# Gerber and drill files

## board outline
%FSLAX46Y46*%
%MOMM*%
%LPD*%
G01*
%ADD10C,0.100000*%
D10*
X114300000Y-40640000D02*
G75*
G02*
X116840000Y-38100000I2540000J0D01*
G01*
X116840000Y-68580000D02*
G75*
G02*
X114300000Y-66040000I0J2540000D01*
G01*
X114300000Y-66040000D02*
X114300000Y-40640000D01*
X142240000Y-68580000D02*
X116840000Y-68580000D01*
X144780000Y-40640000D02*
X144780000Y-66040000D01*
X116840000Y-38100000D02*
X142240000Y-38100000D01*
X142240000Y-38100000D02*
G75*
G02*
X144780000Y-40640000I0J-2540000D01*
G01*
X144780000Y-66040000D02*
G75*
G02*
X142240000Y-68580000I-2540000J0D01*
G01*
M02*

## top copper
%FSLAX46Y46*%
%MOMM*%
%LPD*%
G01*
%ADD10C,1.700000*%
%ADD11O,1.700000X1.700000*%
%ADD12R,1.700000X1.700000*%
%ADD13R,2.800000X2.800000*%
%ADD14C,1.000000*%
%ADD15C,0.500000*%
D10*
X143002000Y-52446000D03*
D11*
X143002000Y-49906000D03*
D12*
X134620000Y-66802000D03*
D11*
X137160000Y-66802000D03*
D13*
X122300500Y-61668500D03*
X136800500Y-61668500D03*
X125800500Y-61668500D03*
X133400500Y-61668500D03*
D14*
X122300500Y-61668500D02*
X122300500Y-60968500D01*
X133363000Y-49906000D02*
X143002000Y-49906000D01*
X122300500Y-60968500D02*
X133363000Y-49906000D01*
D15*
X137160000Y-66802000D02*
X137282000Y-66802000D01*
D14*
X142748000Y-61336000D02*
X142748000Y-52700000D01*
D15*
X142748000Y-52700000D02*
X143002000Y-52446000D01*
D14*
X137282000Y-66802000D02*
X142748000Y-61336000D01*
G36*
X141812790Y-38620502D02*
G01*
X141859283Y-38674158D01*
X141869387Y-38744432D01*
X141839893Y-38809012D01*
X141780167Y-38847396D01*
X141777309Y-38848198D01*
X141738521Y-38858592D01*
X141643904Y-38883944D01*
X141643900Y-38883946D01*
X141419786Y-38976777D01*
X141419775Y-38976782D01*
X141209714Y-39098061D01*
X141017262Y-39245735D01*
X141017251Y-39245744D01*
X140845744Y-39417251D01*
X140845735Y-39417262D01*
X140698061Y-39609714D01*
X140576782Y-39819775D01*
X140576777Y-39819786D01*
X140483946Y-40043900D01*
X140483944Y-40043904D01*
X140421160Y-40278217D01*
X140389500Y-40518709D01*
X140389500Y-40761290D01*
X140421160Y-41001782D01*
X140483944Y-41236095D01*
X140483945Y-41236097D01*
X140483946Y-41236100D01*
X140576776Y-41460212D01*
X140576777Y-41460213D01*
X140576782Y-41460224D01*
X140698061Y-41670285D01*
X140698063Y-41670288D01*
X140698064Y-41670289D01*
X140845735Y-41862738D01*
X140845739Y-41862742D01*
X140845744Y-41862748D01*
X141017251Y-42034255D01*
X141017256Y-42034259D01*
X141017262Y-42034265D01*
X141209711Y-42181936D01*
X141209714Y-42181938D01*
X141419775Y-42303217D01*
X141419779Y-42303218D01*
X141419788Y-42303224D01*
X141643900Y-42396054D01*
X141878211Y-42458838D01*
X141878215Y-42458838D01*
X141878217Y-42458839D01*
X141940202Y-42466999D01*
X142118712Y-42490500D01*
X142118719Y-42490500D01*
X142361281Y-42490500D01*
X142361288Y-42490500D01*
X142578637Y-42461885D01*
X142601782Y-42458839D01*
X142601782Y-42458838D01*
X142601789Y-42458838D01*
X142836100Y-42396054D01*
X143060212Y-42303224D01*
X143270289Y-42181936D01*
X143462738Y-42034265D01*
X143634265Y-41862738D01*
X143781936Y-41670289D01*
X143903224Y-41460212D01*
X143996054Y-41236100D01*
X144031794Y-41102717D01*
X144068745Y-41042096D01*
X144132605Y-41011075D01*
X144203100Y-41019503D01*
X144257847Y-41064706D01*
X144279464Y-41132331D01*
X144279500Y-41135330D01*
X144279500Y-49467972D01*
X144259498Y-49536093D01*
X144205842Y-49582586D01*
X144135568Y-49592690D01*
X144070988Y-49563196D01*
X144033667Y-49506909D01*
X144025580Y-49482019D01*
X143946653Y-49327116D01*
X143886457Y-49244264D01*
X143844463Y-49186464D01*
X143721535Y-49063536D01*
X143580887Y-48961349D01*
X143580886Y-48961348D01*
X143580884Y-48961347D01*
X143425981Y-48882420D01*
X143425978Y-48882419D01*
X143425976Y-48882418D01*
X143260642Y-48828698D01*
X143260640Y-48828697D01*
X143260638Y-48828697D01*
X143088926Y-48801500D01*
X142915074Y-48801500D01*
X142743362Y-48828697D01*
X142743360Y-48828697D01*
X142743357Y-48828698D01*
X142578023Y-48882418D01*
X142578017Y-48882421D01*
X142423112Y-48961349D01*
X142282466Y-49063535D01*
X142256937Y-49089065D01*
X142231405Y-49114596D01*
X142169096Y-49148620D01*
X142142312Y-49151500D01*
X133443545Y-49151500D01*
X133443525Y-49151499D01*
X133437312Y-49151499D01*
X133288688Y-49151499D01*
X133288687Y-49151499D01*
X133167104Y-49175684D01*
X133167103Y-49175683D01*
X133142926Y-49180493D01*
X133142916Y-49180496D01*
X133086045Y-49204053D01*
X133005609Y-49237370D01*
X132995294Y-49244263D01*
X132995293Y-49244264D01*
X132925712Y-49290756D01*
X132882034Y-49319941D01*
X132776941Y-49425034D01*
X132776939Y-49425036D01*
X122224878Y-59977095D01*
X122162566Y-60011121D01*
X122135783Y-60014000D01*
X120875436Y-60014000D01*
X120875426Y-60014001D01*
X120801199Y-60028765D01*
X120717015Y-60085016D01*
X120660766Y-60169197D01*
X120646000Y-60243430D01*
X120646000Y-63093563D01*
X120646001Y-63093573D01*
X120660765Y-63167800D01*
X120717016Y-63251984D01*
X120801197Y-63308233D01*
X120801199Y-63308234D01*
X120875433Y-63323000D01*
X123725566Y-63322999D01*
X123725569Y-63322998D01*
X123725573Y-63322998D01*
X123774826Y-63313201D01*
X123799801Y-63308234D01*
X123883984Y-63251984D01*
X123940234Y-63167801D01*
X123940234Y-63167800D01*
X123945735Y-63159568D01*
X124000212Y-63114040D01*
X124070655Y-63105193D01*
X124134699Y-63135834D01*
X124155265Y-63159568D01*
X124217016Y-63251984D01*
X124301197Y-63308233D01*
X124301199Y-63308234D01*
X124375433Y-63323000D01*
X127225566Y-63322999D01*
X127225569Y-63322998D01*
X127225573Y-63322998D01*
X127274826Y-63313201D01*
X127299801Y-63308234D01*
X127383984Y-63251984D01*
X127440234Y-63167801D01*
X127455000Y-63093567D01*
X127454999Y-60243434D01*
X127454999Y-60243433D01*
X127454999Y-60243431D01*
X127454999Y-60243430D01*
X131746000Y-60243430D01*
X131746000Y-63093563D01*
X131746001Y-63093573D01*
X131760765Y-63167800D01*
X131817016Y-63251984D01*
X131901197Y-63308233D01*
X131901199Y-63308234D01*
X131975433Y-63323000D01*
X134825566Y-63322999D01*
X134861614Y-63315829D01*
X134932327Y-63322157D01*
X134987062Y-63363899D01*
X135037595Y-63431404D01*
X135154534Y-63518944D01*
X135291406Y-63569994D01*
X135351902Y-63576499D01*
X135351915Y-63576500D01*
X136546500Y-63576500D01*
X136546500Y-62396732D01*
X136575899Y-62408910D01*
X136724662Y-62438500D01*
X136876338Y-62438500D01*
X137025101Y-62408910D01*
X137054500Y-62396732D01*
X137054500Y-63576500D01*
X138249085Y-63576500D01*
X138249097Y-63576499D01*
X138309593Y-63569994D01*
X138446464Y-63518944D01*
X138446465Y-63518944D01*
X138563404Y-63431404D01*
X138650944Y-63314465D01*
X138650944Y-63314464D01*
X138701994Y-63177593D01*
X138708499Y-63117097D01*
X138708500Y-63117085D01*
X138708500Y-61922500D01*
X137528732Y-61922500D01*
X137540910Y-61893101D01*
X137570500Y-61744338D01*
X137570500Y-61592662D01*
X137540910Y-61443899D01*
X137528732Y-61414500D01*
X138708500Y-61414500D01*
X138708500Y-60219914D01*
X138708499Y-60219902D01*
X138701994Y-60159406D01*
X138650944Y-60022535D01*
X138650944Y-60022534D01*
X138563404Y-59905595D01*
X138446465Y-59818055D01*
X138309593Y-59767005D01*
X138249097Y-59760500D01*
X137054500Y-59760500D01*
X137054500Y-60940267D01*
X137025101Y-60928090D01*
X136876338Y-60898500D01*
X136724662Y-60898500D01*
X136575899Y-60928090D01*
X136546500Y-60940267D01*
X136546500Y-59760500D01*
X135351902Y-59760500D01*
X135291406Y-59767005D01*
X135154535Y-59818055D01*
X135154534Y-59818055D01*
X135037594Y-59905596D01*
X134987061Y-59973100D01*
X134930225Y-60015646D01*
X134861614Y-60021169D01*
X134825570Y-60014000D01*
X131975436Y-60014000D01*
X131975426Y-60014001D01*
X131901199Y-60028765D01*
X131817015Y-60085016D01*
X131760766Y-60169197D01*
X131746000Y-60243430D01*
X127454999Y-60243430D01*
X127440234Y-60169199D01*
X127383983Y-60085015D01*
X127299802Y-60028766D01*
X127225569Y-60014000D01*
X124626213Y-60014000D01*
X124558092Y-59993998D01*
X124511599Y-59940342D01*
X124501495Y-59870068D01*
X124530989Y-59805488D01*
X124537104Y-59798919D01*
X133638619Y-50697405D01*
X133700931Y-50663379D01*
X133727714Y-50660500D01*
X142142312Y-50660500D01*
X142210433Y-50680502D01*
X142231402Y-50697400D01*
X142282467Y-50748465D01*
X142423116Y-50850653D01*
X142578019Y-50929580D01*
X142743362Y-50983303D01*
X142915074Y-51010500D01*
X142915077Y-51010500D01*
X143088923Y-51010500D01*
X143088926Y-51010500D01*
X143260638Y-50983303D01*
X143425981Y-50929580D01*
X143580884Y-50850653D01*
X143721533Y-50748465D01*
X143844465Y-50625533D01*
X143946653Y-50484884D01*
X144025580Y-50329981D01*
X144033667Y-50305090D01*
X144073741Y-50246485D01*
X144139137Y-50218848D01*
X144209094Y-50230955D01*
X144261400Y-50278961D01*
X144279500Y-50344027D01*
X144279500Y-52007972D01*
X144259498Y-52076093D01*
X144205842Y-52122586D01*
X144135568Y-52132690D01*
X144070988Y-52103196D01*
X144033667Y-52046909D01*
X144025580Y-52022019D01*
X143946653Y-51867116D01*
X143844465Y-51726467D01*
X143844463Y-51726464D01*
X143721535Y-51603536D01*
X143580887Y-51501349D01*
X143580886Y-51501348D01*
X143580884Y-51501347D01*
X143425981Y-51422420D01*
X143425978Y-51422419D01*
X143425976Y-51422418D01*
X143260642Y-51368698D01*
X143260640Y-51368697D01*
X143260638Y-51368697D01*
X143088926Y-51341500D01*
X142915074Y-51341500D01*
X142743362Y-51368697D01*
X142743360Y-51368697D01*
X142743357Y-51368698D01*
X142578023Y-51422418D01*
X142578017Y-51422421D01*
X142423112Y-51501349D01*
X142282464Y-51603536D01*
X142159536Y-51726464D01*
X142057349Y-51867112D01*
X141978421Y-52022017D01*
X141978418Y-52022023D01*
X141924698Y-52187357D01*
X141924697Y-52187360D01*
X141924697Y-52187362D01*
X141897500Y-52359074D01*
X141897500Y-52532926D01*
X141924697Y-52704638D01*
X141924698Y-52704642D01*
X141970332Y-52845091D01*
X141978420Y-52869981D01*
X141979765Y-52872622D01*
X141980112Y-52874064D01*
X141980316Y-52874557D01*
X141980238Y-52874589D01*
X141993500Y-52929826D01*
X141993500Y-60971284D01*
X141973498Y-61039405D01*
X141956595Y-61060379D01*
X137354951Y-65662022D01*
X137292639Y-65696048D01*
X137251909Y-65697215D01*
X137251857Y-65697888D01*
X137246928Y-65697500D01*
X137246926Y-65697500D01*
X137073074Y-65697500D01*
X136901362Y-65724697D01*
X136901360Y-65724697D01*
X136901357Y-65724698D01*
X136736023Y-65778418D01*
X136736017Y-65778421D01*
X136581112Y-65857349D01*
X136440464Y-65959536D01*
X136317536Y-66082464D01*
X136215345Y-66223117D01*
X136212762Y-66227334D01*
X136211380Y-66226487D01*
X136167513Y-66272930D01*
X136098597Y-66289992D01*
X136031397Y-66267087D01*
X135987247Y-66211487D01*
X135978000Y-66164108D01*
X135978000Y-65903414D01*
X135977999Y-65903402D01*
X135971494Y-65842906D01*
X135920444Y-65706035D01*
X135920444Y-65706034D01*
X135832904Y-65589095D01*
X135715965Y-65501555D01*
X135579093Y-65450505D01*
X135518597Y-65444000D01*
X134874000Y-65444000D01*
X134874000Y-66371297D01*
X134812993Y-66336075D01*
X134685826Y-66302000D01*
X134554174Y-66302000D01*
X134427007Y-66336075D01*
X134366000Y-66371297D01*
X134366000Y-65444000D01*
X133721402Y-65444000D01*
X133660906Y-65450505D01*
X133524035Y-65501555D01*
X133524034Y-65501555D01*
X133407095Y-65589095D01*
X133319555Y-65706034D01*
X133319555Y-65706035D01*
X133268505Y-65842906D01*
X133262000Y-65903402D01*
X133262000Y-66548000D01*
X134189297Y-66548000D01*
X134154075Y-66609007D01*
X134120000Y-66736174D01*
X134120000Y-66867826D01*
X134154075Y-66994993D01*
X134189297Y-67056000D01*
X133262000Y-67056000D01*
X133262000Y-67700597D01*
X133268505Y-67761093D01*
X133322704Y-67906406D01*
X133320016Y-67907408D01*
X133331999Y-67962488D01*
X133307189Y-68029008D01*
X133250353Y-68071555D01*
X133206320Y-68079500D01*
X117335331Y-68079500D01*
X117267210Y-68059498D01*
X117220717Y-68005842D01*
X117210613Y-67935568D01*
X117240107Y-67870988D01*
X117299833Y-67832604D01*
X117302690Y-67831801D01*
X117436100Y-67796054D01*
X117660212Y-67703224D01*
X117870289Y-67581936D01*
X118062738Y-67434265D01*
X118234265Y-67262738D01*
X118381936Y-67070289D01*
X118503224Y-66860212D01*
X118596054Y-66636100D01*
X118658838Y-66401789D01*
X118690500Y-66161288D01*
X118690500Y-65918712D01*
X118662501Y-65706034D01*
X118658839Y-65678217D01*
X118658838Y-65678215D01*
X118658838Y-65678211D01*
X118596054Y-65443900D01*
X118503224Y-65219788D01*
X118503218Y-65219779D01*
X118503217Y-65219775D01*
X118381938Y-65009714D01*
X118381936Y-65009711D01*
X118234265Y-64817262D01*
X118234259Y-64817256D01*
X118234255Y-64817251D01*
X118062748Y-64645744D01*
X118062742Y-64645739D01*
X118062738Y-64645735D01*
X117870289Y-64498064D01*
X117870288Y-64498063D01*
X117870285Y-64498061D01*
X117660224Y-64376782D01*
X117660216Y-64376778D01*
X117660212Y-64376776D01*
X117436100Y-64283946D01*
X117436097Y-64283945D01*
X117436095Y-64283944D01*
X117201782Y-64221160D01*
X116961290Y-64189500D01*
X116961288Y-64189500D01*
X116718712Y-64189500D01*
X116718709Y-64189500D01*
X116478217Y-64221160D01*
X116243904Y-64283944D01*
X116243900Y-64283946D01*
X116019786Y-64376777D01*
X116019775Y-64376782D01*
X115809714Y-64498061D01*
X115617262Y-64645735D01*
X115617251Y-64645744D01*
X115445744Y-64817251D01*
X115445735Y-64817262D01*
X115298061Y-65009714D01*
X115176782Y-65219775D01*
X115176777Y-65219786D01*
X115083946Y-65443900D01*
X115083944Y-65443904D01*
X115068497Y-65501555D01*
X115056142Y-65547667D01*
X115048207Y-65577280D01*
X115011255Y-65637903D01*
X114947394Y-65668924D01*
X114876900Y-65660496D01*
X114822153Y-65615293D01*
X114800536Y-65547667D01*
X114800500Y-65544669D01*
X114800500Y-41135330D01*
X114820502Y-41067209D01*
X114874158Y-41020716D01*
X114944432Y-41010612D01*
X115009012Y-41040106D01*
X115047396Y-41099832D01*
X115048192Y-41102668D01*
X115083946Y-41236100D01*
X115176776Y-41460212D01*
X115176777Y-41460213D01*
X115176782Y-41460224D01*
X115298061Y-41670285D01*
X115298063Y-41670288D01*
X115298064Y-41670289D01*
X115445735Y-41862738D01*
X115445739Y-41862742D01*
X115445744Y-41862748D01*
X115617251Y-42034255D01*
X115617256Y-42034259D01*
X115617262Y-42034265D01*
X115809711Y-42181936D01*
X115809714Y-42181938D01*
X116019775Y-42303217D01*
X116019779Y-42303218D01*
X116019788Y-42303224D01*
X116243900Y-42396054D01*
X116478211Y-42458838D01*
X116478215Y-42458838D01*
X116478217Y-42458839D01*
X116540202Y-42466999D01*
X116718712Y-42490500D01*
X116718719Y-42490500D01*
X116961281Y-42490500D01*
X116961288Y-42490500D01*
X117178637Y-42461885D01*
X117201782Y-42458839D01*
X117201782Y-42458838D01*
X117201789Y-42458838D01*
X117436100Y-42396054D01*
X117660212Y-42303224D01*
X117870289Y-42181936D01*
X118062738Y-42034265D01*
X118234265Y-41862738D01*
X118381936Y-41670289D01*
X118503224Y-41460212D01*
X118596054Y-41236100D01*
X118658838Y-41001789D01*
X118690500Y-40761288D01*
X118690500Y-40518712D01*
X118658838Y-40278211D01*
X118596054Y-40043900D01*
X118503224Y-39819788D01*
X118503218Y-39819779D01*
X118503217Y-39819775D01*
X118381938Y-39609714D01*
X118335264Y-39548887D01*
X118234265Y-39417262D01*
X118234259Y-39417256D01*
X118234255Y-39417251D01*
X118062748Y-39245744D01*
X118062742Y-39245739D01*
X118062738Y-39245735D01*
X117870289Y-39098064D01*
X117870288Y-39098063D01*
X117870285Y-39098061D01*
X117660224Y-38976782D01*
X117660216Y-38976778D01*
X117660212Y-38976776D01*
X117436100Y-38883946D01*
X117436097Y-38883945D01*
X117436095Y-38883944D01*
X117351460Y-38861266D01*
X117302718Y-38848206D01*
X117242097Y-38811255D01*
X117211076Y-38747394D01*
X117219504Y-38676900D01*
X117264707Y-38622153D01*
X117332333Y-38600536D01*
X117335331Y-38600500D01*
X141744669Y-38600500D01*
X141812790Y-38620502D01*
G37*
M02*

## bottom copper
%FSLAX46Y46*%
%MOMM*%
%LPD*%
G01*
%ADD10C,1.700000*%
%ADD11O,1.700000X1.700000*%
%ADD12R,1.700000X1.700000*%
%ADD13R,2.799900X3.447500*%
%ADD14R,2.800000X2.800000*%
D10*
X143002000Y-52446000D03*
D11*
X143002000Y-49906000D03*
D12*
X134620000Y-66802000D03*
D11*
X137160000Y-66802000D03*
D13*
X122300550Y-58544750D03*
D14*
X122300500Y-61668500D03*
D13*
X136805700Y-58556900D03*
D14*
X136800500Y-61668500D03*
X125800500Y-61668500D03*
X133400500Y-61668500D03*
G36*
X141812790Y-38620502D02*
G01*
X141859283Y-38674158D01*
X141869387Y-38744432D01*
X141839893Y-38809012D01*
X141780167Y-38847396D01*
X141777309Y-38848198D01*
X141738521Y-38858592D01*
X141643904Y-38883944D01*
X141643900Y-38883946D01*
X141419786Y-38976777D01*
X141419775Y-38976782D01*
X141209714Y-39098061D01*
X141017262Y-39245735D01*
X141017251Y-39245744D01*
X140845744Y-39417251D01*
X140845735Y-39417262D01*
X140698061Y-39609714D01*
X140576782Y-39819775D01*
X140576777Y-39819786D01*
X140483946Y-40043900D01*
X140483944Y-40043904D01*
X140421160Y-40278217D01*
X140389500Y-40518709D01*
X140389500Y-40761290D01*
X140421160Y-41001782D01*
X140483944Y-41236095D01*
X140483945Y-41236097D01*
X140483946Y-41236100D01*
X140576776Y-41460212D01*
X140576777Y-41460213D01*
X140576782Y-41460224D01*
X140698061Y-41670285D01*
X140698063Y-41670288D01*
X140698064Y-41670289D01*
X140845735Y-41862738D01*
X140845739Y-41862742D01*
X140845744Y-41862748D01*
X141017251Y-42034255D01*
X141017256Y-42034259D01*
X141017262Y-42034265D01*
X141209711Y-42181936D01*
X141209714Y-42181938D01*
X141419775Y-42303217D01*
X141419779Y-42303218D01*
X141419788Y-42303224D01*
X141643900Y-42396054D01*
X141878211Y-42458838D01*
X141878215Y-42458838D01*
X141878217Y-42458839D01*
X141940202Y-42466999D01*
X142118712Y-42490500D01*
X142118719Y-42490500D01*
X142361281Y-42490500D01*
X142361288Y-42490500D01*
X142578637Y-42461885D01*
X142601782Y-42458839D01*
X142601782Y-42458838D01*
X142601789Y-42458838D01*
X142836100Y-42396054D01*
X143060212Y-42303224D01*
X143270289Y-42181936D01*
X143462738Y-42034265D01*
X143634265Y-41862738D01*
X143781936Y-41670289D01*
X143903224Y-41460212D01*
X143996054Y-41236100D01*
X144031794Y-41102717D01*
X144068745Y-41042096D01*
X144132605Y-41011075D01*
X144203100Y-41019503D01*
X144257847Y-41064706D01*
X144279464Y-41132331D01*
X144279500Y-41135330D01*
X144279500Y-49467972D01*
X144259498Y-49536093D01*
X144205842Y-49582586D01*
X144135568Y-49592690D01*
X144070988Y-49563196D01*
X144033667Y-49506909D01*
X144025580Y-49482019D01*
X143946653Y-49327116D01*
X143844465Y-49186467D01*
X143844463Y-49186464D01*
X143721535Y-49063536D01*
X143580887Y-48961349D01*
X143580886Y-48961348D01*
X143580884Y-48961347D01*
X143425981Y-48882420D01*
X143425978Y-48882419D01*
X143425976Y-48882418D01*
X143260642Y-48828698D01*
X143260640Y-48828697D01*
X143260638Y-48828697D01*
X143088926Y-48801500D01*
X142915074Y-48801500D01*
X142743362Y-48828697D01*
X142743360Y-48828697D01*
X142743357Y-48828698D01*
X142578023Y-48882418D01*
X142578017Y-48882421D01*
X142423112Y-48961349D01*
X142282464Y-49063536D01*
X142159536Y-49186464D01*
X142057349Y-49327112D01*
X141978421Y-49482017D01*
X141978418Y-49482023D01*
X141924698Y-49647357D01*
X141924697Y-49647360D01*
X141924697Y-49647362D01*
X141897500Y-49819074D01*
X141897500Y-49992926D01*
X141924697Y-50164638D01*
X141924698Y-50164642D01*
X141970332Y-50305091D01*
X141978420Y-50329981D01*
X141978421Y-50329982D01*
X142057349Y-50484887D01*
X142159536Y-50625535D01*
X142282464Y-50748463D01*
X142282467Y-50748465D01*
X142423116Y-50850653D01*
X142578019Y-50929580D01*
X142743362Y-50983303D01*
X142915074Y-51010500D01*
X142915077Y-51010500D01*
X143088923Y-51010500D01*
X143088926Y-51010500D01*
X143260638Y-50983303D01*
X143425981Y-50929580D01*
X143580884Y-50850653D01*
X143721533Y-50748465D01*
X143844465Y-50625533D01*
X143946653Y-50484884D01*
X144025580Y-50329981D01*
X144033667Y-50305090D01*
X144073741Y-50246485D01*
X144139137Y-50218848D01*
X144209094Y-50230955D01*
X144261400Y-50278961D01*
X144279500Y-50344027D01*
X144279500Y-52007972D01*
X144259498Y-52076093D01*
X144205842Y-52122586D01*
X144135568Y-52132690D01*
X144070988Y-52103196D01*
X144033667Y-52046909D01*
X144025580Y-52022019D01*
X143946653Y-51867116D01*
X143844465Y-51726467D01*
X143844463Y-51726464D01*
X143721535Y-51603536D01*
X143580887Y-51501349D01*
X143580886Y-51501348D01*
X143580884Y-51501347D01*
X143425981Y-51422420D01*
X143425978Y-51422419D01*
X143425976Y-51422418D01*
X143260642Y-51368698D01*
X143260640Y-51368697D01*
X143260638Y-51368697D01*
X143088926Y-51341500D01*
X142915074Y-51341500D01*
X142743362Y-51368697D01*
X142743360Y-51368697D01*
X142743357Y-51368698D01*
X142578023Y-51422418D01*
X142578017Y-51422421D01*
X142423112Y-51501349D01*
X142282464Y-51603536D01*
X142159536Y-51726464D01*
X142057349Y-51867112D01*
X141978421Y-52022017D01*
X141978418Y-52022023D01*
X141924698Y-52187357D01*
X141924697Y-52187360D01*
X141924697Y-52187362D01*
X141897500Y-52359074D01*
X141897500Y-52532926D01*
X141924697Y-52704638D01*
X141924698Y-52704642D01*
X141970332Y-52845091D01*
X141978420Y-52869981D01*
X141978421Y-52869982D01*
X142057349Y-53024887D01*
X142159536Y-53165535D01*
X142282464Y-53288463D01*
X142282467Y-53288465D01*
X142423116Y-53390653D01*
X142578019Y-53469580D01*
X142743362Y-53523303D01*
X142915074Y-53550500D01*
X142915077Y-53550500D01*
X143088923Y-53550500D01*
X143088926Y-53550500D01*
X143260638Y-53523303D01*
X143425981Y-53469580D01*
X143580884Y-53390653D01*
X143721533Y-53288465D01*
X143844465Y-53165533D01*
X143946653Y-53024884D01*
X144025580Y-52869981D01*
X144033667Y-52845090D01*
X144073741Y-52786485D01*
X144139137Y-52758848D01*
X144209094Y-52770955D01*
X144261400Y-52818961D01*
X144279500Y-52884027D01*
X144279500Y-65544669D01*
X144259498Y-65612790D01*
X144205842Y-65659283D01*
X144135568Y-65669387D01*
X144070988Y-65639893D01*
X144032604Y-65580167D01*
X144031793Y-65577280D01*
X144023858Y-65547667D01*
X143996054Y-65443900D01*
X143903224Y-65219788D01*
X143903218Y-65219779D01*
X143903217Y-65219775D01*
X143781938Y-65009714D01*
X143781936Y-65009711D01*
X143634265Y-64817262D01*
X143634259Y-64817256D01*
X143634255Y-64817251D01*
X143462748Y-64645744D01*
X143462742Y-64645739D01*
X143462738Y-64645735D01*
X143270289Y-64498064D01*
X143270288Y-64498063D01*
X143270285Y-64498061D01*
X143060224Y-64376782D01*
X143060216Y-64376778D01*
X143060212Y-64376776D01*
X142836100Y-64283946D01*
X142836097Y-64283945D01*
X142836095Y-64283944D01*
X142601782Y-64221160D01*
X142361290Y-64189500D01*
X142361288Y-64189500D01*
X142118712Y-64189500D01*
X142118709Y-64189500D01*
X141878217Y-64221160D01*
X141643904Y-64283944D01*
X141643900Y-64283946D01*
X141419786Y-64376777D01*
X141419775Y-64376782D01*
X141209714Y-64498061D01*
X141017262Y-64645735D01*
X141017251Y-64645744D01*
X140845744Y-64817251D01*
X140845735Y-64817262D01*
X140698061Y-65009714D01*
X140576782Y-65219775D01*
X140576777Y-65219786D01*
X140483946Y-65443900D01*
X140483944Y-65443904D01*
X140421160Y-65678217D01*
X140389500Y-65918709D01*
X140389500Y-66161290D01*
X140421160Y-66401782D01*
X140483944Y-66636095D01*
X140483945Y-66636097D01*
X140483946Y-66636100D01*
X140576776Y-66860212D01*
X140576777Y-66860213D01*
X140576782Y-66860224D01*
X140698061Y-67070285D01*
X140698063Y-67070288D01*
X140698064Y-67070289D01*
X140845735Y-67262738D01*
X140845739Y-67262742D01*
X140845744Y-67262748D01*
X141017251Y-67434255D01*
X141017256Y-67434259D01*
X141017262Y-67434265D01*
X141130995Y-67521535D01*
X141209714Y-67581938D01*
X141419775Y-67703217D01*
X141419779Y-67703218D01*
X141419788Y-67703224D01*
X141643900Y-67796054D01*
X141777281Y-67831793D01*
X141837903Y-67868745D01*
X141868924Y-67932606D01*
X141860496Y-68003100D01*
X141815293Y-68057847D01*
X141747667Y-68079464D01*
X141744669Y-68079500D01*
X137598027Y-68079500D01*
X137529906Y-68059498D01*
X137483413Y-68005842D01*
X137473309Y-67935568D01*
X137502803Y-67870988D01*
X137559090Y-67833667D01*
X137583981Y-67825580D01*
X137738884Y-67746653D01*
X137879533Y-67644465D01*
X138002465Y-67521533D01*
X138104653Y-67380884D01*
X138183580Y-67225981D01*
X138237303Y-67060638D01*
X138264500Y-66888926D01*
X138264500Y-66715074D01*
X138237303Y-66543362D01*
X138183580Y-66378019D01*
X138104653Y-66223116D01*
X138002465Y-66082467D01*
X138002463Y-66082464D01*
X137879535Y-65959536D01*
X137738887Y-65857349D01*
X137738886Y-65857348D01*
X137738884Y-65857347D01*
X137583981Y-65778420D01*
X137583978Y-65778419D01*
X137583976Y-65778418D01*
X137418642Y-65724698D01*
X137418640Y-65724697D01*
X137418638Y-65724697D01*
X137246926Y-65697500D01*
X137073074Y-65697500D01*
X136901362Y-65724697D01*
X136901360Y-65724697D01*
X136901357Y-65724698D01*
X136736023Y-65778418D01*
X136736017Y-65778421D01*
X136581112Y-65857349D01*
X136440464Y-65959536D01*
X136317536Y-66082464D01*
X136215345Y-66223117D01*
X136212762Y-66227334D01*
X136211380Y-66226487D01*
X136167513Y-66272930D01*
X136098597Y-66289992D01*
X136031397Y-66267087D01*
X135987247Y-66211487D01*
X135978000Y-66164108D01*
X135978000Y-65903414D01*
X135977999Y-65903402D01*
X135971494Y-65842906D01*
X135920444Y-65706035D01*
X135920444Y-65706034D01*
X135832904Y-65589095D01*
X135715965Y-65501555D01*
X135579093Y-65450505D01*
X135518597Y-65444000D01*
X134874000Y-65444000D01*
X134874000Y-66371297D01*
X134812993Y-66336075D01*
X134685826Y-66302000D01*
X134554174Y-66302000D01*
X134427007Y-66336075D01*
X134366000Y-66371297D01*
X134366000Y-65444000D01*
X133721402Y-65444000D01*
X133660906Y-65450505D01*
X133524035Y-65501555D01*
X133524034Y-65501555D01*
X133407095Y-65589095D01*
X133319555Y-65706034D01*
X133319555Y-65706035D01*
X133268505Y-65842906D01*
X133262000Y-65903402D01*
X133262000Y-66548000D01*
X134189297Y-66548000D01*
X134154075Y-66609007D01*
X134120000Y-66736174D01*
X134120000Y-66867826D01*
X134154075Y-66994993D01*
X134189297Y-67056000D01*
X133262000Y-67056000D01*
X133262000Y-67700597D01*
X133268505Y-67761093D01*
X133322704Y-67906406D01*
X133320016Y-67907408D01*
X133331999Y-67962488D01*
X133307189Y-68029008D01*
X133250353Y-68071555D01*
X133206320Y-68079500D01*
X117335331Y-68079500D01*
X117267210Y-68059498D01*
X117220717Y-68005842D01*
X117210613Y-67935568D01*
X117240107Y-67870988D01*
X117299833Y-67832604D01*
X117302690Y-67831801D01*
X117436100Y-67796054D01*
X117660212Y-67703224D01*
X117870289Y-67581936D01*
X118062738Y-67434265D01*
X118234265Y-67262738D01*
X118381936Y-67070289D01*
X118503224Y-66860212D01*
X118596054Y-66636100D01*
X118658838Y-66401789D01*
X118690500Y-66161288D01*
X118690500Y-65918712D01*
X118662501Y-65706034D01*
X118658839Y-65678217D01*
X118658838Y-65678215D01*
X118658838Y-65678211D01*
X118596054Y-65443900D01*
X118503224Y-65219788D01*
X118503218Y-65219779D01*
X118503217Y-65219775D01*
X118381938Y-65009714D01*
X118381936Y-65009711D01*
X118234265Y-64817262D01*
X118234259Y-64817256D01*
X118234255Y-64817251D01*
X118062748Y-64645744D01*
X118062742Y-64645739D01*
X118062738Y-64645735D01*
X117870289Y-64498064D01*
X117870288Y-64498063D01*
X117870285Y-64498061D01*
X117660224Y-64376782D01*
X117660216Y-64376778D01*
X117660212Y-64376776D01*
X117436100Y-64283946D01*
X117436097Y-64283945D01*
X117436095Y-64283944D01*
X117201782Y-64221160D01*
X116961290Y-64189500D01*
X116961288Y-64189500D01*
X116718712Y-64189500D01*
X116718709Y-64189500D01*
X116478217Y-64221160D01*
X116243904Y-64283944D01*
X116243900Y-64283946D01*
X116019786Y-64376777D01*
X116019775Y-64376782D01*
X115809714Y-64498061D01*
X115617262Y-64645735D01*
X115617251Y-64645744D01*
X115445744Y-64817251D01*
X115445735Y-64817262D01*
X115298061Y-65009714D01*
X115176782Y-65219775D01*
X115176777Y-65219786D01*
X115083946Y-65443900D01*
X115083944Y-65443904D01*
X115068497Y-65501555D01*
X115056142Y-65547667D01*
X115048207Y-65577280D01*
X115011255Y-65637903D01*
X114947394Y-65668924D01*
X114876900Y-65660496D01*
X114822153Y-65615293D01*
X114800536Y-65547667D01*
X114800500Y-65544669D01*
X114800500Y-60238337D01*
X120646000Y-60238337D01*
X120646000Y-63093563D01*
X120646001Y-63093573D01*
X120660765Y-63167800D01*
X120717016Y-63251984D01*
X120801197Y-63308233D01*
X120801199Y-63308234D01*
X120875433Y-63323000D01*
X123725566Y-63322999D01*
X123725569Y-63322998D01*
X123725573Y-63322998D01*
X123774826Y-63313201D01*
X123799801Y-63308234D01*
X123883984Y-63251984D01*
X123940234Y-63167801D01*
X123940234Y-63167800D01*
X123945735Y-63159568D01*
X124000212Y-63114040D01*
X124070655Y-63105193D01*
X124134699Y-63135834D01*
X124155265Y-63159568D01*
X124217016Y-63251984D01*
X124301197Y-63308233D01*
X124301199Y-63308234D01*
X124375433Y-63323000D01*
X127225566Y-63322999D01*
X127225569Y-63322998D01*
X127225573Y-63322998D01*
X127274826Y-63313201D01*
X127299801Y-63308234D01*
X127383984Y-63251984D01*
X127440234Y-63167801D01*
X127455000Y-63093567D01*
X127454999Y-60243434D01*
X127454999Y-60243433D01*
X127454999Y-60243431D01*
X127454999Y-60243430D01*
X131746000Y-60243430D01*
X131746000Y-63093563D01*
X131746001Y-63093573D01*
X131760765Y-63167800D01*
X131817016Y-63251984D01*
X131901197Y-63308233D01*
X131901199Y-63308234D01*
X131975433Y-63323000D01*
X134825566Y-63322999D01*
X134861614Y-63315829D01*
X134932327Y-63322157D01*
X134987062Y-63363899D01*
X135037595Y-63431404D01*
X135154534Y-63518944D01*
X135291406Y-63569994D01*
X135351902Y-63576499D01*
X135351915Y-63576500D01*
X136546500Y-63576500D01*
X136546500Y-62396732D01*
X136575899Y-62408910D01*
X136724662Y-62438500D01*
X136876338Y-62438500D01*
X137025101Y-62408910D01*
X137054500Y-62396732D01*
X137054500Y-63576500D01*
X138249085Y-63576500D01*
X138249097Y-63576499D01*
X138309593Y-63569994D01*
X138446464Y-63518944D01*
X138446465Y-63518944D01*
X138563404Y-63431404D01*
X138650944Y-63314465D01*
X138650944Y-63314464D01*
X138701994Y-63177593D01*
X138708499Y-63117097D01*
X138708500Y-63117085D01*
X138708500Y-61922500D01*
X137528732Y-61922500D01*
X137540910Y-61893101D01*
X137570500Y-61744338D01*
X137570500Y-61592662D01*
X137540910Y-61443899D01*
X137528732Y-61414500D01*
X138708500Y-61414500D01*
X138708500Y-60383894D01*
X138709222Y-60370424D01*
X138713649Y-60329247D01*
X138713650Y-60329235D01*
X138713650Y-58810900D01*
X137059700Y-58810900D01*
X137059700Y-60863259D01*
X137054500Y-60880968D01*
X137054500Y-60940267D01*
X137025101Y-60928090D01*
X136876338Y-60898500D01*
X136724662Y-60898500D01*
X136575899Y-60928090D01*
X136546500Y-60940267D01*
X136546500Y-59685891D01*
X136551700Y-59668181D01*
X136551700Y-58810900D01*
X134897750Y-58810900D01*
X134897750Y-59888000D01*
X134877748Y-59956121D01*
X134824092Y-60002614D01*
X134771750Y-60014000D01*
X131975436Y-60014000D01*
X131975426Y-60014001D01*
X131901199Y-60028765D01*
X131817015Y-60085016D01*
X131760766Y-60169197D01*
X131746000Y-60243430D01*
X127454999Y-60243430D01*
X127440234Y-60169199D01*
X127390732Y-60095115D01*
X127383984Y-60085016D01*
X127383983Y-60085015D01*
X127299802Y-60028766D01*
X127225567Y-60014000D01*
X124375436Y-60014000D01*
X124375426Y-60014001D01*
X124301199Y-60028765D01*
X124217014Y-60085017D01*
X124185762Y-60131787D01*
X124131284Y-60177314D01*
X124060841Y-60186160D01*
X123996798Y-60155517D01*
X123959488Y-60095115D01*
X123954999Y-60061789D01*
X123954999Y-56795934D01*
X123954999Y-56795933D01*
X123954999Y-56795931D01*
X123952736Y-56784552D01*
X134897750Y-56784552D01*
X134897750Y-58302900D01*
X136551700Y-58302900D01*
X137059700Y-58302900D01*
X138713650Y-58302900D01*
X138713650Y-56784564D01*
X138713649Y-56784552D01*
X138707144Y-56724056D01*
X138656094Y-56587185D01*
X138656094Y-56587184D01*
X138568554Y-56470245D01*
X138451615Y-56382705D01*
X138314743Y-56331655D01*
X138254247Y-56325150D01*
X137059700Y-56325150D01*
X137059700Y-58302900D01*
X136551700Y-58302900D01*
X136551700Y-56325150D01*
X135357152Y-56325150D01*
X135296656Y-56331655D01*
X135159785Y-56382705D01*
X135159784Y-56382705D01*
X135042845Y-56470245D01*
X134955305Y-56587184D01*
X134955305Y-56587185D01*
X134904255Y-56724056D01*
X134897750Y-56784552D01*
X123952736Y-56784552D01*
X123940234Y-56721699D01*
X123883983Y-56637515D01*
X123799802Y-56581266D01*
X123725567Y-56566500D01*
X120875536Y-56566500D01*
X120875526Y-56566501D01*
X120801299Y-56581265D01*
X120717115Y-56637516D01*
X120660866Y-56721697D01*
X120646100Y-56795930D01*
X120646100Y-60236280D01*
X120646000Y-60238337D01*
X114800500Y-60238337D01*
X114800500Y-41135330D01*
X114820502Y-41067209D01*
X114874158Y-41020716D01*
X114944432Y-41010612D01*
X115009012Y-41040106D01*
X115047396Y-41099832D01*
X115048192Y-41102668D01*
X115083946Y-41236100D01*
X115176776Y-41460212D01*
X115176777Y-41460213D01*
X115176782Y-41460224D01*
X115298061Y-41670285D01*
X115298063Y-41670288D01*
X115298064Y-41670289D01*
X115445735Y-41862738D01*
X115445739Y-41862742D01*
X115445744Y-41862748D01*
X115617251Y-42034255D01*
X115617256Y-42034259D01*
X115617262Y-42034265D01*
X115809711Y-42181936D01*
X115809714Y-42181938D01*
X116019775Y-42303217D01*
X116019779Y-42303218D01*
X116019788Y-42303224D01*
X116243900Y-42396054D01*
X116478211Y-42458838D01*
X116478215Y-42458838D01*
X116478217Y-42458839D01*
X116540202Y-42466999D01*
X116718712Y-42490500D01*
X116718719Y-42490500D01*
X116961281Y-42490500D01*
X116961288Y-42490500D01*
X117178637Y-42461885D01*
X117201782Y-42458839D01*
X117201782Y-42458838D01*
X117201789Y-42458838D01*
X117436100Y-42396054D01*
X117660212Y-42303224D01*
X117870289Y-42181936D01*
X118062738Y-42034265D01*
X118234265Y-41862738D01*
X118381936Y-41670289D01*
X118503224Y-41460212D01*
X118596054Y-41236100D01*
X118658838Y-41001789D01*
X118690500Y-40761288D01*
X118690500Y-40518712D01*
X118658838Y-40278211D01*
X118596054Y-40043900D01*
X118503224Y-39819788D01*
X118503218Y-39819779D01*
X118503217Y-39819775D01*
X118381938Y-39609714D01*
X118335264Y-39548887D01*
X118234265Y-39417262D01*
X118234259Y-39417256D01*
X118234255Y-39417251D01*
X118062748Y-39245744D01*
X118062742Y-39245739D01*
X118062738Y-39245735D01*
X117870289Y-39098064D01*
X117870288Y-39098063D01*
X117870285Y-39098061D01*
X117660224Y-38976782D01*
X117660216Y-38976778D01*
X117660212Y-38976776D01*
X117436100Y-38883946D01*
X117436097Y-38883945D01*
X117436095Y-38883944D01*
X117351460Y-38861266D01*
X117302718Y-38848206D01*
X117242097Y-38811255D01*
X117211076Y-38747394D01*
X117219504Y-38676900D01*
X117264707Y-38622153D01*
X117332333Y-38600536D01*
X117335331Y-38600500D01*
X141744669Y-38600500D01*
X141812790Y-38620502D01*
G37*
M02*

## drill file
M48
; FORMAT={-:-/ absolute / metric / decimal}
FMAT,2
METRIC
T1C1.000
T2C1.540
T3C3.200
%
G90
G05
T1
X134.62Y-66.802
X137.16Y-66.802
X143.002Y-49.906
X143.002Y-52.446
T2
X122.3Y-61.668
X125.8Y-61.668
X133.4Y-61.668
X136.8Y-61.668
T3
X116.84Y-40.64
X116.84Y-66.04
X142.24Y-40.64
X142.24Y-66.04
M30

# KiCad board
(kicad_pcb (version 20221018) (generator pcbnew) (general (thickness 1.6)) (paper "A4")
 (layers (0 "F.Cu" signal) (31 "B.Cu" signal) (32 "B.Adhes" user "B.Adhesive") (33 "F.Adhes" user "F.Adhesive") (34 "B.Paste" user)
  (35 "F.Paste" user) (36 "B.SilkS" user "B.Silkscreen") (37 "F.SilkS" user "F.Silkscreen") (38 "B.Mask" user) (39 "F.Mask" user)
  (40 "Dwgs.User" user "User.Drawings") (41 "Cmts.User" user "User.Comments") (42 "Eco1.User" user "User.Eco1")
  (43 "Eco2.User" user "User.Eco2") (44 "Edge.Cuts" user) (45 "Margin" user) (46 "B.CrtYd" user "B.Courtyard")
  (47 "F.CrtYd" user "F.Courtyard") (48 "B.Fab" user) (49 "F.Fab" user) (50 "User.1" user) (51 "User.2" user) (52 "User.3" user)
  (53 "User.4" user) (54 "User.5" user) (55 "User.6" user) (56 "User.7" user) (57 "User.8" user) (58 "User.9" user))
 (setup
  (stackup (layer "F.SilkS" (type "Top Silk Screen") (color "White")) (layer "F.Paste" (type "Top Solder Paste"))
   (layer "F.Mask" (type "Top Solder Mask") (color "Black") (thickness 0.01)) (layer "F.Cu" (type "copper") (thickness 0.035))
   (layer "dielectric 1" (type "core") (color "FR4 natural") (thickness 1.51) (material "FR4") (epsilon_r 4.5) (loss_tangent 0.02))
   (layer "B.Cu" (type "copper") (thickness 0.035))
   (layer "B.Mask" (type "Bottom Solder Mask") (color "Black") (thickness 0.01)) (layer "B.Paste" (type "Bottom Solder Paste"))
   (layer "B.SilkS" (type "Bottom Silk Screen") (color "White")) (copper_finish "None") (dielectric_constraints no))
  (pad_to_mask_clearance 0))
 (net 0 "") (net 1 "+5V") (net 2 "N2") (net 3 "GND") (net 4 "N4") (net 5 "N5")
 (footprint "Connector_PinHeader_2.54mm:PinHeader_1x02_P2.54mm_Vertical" (layer "F.Cu") (at 143.002 52.446 180)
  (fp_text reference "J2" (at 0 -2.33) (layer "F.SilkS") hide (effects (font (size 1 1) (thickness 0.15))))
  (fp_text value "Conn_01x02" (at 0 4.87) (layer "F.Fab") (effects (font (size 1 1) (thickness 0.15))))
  (pad "1" thru_hole circle (at 0 0 180) (size 1.7 1.7) (drill 1) (layers "*.Cu" "*.Mask") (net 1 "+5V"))
  (pad "2" thru_hole oval (at 0 2.54 180) (size 1.7 1.7) (drill 1) (layers "*.Cu" "*.Mask") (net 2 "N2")))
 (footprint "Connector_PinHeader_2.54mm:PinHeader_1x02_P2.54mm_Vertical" (layer "F.Cu") (at 134.62 66.802 90)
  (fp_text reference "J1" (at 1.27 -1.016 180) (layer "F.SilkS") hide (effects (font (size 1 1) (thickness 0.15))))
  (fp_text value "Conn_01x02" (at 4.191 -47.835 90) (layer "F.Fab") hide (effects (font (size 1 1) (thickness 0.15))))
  (pad "1" thru_hole rect (at 0 0 90) (size 1.7 1.7) (drill 1) (layers "*.Cu" "*.Mask") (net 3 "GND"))
  (pad "2" thru_hole oval (at 0 2.54 90) (size 1.7 1.7) (drill 1) (layers "*.Cu" "*.Mask") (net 1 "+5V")))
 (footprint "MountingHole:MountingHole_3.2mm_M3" (layer "F.Cu") (at 142.24 40.64)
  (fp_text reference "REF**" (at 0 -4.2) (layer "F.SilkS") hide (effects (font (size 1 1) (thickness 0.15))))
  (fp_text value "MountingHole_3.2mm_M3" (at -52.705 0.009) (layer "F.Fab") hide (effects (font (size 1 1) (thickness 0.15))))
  (pad "" np_thru_hole circle (at 0 0) (size 3.2 3.2) (drill 3.2) (layers "*.Cu" "*.Mask")))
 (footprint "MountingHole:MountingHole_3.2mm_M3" (layer "F.Cu") (at 142.24 66.04)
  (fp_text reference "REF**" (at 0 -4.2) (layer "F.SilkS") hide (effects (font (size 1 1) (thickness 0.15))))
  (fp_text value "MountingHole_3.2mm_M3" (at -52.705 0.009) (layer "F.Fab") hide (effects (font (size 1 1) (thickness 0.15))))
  (pad "" np_thru_hole circle (at 0 0) (size 3.2 3.2) (drill 3.2) (layers "*.Cu" "*.Mask")))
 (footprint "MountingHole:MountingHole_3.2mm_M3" (layer "F.Cu") (at 116.84 40.64)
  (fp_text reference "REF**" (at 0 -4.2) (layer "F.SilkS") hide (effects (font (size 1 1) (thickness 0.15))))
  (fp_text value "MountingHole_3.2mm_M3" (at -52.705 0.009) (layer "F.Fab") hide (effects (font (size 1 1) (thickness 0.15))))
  (pad "" np_thru_hole circle (at 0 0) (size 3.2 3.2) (drill 3.2) (layers "*.Cu" "*.Mask")))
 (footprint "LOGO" (layer "F.Cu") (at 129.54 52.832)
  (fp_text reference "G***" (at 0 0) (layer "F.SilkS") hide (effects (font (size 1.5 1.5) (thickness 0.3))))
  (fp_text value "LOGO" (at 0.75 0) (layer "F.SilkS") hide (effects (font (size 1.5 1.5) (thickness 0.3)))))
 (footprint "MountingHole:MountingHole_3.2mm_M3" (layer "F.Cu") (at 116.84 66.04)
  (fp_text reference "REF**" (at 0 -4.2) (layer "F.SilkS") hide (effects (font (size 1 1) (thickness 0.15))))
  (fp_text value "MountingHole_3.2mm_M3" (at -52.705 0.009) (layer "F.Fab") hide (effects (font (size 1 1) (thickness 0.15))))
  (pad "" np_thru_hole circle (at 0 0) (size 3.2 3.2) (drill 3.2) (layers "*.Cu" "*.Mask")))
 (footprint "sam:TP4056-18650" (layer "B.Cu") (at 120.6005 37.0685 -90)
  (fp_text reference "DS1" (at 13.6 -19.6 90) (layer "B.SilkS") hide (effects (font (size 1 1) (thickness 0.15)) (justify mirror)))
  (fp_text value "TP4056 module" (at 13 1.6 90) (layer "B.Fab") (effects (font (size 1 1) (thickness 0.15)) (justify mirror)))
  (pad "3" smd rect (at 21.47625 -1.70005 270) (size 3.4475 2.7999) (layers "B.Cu" "B.Paste" "B.Mask") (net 2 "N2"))
  (pad "3" thru_hole rect (at 24.6 -1.7 270) (size 2.8 2.8) (drill 1.54) (layers "*.Cu" "*.Mask") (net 2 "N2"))
  (pad "4" smd rect (at 21.4884 -16.2052 270) (size 3.4475 2.7999) (layers "B.Cu" "B.Paste" "B.Mask") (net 3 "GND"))
  (pad "4" thru_hole rect (at 24.6 -16.2 270) (size 2.8 2.8) (drill 1.54) (layers "*.Cu" "*.Mask") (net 3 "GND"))
  (pad "5" thru_hole rect (at 24.6 -5.2 270) (size 2.8 2.8) (drill 1.54) (layers "*.Cu" "*.Mask") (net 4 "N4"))
  (pad "6" thru_hole rect (at 24.6 -12.8 270) (size 2.8 2.8) (drill 1.54) (layers "*.Cu" "*.Mask") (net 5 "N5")))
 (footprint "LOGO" (layer "B.Cu") (at 129.54 49.784 180)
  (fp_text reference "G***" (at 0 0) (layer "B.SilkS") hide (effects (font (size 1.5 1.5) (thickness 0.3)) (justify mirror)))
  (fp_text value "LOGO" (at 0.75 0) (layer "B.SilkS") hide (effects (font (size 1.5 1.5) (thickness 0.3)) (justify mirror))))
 (gr_arc (start 114.3 40.64) (mid 115.043949 38.843949) (end 116.84 38.1) (stroke (width 0.1) (type default)) (layer "Edge.Cuts"))
 (gr_arc (start 116.84 68.58) (mid 115.043949 67.836051) (end 114.3 66.04) (stroke (width 0.1) (type default)) (layer "Edge.Cuts"))
 (gr_line (start 114.3 66.04) (end 114.3 40.64) (stroke (width 0.1) (type default)) (layer "Edge.Cuts"))
 (gr_line (start 142.24 68.58) (end 116.84 68.58) (stroke (width 0.1) (type default)) (layer "Edge.Cuts"))
 (gr_line (start 144.78 40.64) (end 144.78 66.04) (stroke (width 0.1) (type default)) (layer "Edge.Cuts"))
 (gr_line (start 116.84 38.1) (end 142.24 38.1) (stroke (width 0.1) (type default)) (layer "Edge.Cuts"))
 (gr_arc (start 142.24 38.1) (mid 144.036051 38.843949) (end 144.78 40.64) (stroke (width 0.1) (type default)) (layer "Edge.Cuts"))
 (gr_arc (start 144.78 66.04) (mid 144.036051 67.836051) (end 142.24 68.58) (stroke (width 0.1) (type default)) (layer "Edge.Cuts"))
 (segment (start 122.3005 61.6685) (end 122.3005 60.9685) (width 1) (layer "F.Cu") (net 2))
 (segment (start 133.363 49.906) (end 143.002 49.906) (width 1) (layer "F.Cu") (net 2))
 (segment (start 122.3005 60.9685) (end 133.363 49.906) (width 1) (layer "F.Cu") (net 2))
 (segment (start 137.16 66.802) (end 137.282 66.802) (width 0.5) (layer "F.Cu") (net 1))
 (segment (start 142.748 61.336) (end 142.748 52.7) (width 1) (layer "F.Cu") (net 1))
 (segment (start 142.748 52.7) (end 143.002 52.446) (width 0.5) (layer "F.Cu") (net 1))
 (segment (start 137.282 66.802) (end 142.748 61.336) (width 1) (layer "F.Cu") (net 1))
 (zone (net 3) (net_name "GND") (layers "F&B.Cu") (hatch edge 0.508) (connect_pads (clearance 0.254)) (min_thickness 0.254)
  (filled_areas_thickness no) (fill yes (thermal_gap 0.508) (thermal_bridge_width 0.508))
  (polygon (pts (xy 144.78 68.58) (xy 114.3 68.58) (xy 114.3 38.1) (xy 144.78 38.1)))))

